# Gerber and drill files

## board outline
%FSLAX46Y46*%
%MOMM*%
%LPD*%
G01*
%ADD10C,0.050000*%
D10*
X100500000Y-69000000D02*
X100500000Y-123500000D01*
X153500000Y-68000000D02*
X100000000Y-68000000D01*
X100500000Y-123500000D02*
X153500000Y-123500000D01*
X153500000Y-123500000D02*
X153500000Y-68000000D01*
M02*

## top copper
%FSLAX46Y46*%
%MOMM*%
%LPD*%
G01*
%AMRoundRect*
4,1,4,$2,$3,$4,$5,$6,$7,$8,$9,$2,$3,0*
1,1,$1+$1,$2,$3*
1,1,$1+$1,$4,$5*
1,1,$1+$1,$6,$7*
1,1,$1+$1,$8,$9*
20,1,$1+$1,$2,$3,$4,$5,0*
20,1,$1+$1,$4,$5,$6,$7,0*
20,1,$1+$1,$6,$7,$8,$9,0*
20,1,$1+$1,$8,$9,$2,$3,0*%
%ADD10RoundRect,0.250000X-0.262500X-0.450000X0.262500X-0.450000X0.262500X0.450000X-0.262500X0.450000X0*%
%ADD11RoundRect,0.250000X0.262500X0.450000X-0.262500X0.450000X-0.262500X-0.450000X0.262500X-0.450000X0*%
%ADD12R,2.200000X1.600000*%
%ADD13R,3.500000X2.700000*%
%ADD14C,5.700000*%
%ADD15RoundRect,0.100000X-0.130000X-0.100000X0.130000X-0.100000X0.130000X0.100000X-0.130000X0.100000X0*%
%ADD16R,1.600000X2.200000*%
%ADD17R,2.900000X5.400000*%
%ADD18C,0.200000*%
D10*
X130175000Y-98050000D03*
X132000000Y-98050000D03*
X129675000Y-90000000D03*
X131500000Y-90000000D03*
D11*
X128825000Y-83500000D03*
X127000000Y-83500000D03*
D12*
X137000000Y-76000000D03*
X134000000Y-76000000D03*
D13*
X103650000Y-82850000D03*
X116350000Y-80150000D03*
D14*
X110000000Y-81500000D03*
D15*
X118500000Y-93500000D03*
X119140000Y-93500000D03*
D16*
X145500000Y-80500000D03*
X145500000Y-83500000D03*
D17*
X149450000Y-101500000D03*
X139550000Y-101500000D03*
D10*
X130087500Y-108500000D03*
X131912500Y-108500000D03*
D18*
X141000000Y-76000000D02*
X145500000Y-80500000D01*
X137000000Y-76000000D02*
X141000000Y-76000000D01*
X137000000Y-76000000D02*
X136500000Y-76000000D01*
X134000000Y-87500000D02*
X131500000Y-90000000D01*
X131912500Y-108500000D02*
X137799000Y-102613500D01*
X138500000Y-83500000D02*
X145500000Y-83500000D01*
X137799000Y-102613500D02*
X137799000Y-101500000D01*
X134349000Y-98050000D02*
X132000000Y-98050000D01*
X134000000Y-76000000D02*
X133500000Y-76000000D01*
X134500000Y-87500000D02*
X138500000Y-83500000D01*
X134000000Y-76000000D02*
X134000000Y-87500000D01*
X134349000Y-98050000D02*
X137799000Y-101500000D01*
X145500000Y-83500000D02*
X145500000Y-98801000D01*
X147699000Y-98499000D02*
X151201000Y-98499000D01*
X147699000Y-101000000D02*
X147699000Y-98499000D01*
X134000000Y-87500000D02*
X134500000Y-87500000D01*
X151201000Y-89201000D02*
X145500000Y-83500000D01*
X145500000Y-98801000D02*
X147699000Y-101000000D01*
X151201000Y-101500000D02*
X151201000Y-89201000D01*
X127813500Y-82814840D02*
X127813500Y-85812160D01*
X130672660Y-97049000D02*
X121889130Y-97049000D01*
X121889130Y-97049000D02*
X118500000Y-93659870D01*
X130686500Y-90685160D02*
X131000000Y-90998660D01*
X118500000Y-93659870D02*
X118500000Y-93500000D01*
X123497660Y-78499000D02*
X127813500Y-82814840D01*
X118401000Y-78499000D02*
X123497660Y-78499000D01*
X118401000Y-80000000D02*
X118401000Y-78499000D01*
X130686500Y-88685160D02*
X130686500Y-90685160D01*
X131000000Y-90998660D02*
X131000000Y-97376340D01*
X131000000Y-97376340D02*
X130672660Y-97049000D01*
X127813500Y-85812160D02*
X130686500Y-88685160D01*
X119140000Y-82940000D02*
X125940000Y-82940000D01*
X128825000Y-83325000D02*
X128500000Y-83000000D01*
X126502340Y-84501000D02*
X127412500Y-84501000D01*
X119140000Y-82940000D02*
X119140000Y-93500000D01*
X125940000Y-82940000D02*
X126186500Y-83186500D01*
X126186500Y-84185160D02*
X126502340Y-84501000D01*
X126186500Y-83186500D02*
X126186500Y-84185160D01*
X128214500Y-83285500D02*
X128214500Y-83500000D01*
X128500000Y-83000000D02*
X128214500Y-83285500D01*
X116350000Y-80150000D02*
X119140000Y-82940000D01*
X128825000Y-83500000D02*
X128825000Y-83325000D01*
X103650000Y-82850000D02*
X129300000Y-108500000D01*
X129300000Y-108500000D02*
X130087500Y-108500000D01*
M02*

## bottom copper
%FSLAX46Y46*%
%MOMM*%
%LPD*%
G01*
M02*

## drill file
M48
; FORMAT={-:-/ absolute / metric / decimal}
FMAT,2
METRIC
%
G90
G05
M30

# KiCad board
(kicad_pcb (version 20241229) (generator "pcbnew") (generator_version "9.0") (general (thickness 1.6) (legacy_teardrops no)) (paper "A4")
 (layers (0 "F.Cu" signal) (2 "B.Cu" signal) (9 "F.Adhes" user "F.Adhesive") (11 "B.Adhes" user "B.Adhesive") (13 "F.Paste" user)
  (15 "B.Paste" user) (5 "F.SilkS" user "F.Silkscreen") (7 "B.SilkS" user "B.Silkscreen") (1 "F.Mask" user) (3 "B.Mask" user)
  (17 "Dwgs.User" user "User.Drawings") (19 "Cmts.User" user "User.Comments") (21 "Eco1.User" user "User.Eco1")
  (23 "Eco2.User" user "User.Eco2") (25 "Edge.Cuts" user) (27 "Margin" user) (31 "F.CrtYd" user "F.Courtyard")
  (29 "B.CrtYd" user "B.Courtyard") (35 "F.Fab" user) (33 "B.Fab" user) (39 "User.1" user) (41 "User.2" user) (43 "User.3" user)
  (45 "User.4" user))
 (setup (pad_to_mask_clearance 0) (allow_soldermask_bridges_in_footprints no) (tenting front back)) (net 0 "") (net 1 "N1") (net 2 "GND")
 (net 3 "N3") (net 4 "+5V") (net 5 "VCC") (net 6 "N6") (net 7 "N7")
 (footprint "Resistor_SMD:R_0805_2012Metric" (layer "F.Cu") (at 131.0875 98.05)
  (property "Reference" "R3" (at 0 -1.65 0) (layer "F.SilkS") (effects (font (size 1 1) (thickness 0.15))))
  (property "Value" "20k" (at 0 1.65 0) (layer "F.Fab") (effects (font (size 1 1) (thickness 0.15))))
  (pad "1" smd roundrect (at -0.9125 0) (size 1.025 1.4) (layers "F.Cu" "F.Mask" "F.Paste") (roundrect_rratio 0.243902) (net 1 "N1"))
  (pad "2" smd roundrect (at 0.9125 0) (size 1.025 1.4) (layers "F.Cu" "F.Mask" "F.Paste") (roundrect_rratio 0.243902) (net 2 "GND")))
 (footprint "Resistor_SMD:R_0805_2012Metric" (layer "F.Cu") (at 130.5875 90)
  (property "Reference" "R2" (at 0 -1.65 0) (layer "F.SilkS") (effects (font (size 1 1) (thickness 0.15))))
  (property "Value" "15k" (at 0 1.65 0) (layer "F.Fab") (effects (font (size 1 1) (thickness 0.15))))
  (pad "1" smd roundrect (at -0.9125 0) (size 1.025 1.4) (layers "F.Cu" "F.Mask" "F.Paste") (roundrect_rratio 0.243902) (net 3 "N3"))
  (pad "2" smd roundrect (at 0.9125 0) (size 1.025 1.4) (layers "F.Cu" "F.Mask" "F.Paste") (roundrect_rratio 0.243902) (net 2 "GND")))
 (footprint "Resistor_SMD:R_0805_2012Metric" (layer "F.Cu") (at 127.9125 83.5 180)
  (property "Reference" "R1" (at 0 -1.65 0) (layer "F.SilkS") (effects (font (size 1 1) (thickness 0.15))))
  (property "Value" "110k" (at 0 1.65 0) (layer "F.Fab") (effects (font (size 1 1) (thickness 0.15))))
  (pad "1" smd roundrect (at -0.9125 0 180) (size 1.025 1.4) (layers "F.Cu" "F.Mask" "F.Paste") (roundrect_rratio 0.243902) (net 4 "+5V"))
  (pad "2" smd roundrect (at 0.9125 0 180) (size 1.025 1.4) (layers "F.Cu" "F.Mask" "F.Paste") (roundrect_rratio 0.243902) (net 3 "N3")))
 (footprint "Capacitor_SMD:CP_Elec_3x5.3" (layer "F.Cu") (at 135.5 76 180)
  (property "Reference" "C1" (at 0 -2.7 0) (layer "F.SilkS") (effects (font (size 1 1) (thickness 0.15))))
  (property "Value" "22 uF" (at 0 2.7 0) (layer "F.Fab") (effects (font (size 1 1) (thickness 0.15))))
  (pad "1" smd rect (at -1.5 0 180) (size 2.2 1.6) (layers "F.Cu" "F.Mask" "F.Paste") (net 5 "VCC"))
  (pad "2" smd rect (at 1.5 0 180) (size 2.2 1.6) (layers "F.Cu" "F.Mask" "F.Paste") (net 2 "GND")))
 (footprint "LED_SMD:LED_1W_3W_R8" (layer "F.Cu") (at 110 81.5)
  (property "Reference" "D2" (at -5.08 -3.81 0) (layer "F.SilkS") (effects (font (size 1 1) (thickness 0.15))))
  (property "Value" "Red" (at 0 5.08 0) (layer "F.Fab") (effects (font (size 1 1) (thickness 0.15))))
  (pad "1" smd rect (at -6.35 1.35) (size 3.5 2.7) (layers "F.Cu" "F.Mask" "F.Paste") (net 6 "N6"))
  (pad "2" smd rect (at 6.35 -1.35) (size 3.5 2.7) (layers "F.Cu" "F.Mask" "F.Paste") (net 4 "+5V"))
  (pad "3" smd circle (at 0 0) (size 5.7 5.7) (layers "F.Cu" "F.Mask" "F.Paste")))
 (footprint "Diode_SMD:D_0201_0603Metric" (layer "F.Cu") (at 118.82 93.5)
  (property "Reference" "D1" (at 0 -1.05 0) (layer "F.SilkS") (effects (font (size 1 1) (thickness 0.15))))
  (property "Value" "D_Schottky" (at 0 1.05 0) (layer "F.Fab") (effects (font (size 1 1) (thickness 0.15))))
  (pad "" smd roundrect (at -0.345 0) (size 0.318 0.36) (layers "F.Paste") (roundrect_rratio 0.25))
  (pad "" smd roundrect (at 0.345 0) (size 0.318 0.36) (layers "F.Paste") (roundrect_rratio 0.25))
  (pad "1" smd roundrect (at -0.32 0) (size 0.46 0.4) (layers "F.Cu" "F.Mask") (roundrect_rratio 0.25) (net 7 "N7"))
  (pad "2" smd roundrect (at 0.32 0) (size 0.46 0.4) (layers "F.Cu" "F.Mask") (roundrect_rratio 0.25) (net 4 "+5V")))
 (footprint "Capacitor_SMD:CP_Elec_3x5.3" (layer "F.Cu") (at 145.5 82 -90)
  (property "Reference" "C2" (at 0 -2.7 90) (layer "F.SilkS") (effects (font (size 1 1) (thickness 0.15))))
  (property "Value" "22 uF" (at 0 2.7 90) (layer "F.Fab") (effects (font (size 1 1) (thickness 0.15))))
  (pad "1" smd rect (at -1.5 0 270) (size 2.2 1.6) (layers "F.Cu" "F.Mask" "F.Paste") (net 5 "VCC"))
  (pad "2" smd rect (at 1.5 0 270) (size 2.2 1.6) (layers "F.Cu" "F.Mask" "F.Paste") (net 2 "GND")))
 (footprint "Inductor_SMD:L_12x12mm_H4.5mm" (layer "F.Cu") (at 144.5 101.5 180)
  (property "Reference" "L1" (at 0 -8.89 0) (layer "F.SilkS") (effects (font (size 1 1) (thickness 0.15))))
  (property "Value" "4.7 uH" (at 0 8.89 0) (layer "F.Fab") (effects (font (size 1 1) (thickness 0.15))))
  (pad "1" smd rect (at -4.95 0 180) (size 2.9 5.4) (layers "F.Cu" "F.Mask" "F.Paste") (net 5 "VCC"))
  (pad "2" smd rect (at 4.95 0 180) (size 2.9 5.4) (layers "F.Cu" "F.Mask" "F.Paste") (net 7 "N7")))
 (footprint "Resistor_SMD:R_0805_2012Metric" (layer "F.Cu") (at 131 108.5)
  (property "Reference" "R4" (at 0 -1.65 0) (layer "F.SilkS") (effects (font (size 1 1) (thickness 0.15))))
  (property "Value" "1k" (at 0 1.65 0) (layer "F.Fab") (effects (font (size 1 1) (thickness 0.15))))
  (pad "1" smd roundrect (at -0.9125 0) (size 1.025 1.4) (layers "F.Cu" "F.Mask" "F.Paste") (roundrect_rratio 0.243902) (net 6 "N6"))
  (pad "2" smd roundrect (at 0.9125 0) (size 1.025 1.4) (layers "F.Cu" "F.Mask" "F.Paste") (roundrect_rratio 0.243902) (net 2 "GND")))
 (gr_line (start 100.5 69) (end 100.5 123.5) (stroke (width 0.05) (type default)) (layer "Edge.Cuts"))
 (gr_line (start 153.5 68) (end 100 68) (stroke (width 0.05) (type default)) (layer "Edge.Cuts"))
 (gr_line (start 100.5 123.5) (end 153.5 123.5) (stroke (width 0.05) (type default)) (layer "Edge.Cuts"))
 (gr_line (start 153.5 123.5) (end 153.5 68) (stroke (width 0.05) (type default)) (layer "Edge.Cuts"))
 (segment (start 141 76) (end 145.5 80.5) (width 0.2) (layer "F.Cu") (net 5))
 (segment (start 137 76) (end 141 76) (width 0.2) (layer "F.Cu") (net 5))
 (segment (start 137 76) (end 136.5 76) (width 0.2) (layer "F.Cu") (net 5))
 (segment (start 134 87.5) (end 131.5 90) (width 0.2) (layer "F.Cu") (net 2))
 (segment (start 131.9125 108.5) (end 137.799 102.6135) (width 0.2) (layer "F.Cu") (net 2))
 (segment (start 138.5 83.5) (end 145.5 83.5) (width 0.2) (layer "F.Cu") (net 2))
 (segment (start 137.799 102.6135) (end 137.799 101.5) (width 0.2) (layer "F.Cu") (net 2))
 (segment (start 134.349 98.05) (end 132 98.05) (width 0.2) (layer "F.Cu") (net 2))
 (segment (start 134 76) (end 133.5 76) (width 0.2) (layer "F.Cu") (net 2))
 (segment (start 134.5 87.5) (end 138.5 83.5) (width 0.2) (layer "F.Cu") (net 2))
 (segment (start 134 76) (end 134 87.5) (width 0.2) (layer "F.Cu") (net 2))
 (segment (start 134.349 98.05) (end 137.799 101.5) (width 0.2) (layer "F.Cu") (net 2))
 (segment (start 145.5 83.5) (end 145.5 98.801) (width 0.2) (layer "F.Cu") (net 2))
 (segment (start 147.699 98.499) (end 151.201 98.499) (width 0.2) (layer "F.Cu") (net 2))
 (segment (start 147.699 101) (end 147.699 98.499) (width 0.2) (layer "F.Cu") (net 2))
 (segment (start 134 87.5) (end 134.5 87.5) (width 0.2) (layer "F.Cu") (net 2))
 (segment (start 151.201 89.201) (end 145.5 83.5) (width 0.2) (layer "F.Cu") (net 2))
 (segment (start 145.5 98.801) (end 147.699 101) (width 0.2) (layer "F.Cu") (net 2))
 (segment (start 151.201 101.5) (end 151.201 89.201) (width 0.2) (layer "F.Cu") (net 2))
 (segment (start 127.8135 82.81484) (end 127.8135 85.81216) (width 0.2) (layer "F.Cu") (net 7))
 (segment (start 130.67266 97.049) (end 121.88913 97.049) (width 0.2) (layer "F.Cu") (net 7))
 (segment (start 121.88913 97.049) (end 118.5 93.65987) (width 0.2) (layer "F.Cu") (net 7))
 (segment (start 130.6865 90.68516) (end 131 90.99866) (width 0.2) (layer "F.Cu") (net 7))
 (segment (start 118.5 93.65987) (end 118.5 93.5) (width 0.2) (layer "F.Cu") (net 7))
 (segment (start 123.49766 78.499) (end 127.8135 82.81484) (width 0.2) (layer "F.Cu") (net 7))
 (segment (start 118.401 78.499) (end 123.49766 78.499) (width 0.2) (layer "F.Cu") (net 7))
 (segment (start 118.401 80) (end 118.401 78.499) (width 0.2) (layer "F.Cu") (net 7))
 (segment (start 130.6865 88.68516) (end 130.6865 90.68516) (width 0.2) (layer "F.Cu") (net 7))
 (segment (start 131 90.99866) (end 131 97.37634) (width 0.2) (layer "F.Cu") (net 7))
 (segment (start 131 97.37634) (end 130.67266 97.049) (width 0.2) (layer "F.Cu") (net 7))
 (segment (start 127.8135 85.81216) (end 130.6865 88.68516) (width 0.2) (layer "F.Cu") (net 7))
 (segment (start 119.14 82.94) (end 125.94 82.94) (width 0.2) (layer "F.Cu") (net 4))
 (segment (start 128.825 83.325) (end 128.5 83) (width 0.2) (layer "F.Cu") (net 4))
 (segment (start 126.50234 84.501) (end 127.4125 84.501) (width 0.2) (layer "F.Cu") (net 4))
 (segment (start 119.14 82.94) (end 119.14 93.5) (width 0.2) (layer "F.Cu") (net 4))
 (segment (start 125.94 82.94) (end 126.1865 83.1865) (width 0.2) (layer "F.Cu") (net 4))
 (segment (start 126.1865 84.18516) (end 126.50234 84.501) (width 0.2) (layer "F.Cu") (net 4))
 (segment (start 126.1865 83.1865) (end 126.1865 84.18516) (width 0.2) (layer "F.Cu") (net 4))
 (segment (start 128.2145 83.2855) (end 128.2145 83.5) (width 0.2) (layer "F.Cu") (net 4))
 (segment (start 128.5 83) (end 128.2145 83.2855) (width 0.2) (layer "F.Cu") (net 4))
 (segment (start 116.35 80.15) (end 119.14 82.94) (width 0.2) (layer "F.Cu") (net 4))
 (segment (start 128.825 83.5) (end 128.825 83.325) (width 0.2) (layer "F.Cu") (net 4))
 (segment (start 103.65 82.85) (end 129.3 108.5) (width 0.2) (layer "F.Cu") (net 6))
 (segment (start 129.3 108.5) (end 130.0875 108.5) (width 0.2) (layer "F.Cu") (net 6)))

